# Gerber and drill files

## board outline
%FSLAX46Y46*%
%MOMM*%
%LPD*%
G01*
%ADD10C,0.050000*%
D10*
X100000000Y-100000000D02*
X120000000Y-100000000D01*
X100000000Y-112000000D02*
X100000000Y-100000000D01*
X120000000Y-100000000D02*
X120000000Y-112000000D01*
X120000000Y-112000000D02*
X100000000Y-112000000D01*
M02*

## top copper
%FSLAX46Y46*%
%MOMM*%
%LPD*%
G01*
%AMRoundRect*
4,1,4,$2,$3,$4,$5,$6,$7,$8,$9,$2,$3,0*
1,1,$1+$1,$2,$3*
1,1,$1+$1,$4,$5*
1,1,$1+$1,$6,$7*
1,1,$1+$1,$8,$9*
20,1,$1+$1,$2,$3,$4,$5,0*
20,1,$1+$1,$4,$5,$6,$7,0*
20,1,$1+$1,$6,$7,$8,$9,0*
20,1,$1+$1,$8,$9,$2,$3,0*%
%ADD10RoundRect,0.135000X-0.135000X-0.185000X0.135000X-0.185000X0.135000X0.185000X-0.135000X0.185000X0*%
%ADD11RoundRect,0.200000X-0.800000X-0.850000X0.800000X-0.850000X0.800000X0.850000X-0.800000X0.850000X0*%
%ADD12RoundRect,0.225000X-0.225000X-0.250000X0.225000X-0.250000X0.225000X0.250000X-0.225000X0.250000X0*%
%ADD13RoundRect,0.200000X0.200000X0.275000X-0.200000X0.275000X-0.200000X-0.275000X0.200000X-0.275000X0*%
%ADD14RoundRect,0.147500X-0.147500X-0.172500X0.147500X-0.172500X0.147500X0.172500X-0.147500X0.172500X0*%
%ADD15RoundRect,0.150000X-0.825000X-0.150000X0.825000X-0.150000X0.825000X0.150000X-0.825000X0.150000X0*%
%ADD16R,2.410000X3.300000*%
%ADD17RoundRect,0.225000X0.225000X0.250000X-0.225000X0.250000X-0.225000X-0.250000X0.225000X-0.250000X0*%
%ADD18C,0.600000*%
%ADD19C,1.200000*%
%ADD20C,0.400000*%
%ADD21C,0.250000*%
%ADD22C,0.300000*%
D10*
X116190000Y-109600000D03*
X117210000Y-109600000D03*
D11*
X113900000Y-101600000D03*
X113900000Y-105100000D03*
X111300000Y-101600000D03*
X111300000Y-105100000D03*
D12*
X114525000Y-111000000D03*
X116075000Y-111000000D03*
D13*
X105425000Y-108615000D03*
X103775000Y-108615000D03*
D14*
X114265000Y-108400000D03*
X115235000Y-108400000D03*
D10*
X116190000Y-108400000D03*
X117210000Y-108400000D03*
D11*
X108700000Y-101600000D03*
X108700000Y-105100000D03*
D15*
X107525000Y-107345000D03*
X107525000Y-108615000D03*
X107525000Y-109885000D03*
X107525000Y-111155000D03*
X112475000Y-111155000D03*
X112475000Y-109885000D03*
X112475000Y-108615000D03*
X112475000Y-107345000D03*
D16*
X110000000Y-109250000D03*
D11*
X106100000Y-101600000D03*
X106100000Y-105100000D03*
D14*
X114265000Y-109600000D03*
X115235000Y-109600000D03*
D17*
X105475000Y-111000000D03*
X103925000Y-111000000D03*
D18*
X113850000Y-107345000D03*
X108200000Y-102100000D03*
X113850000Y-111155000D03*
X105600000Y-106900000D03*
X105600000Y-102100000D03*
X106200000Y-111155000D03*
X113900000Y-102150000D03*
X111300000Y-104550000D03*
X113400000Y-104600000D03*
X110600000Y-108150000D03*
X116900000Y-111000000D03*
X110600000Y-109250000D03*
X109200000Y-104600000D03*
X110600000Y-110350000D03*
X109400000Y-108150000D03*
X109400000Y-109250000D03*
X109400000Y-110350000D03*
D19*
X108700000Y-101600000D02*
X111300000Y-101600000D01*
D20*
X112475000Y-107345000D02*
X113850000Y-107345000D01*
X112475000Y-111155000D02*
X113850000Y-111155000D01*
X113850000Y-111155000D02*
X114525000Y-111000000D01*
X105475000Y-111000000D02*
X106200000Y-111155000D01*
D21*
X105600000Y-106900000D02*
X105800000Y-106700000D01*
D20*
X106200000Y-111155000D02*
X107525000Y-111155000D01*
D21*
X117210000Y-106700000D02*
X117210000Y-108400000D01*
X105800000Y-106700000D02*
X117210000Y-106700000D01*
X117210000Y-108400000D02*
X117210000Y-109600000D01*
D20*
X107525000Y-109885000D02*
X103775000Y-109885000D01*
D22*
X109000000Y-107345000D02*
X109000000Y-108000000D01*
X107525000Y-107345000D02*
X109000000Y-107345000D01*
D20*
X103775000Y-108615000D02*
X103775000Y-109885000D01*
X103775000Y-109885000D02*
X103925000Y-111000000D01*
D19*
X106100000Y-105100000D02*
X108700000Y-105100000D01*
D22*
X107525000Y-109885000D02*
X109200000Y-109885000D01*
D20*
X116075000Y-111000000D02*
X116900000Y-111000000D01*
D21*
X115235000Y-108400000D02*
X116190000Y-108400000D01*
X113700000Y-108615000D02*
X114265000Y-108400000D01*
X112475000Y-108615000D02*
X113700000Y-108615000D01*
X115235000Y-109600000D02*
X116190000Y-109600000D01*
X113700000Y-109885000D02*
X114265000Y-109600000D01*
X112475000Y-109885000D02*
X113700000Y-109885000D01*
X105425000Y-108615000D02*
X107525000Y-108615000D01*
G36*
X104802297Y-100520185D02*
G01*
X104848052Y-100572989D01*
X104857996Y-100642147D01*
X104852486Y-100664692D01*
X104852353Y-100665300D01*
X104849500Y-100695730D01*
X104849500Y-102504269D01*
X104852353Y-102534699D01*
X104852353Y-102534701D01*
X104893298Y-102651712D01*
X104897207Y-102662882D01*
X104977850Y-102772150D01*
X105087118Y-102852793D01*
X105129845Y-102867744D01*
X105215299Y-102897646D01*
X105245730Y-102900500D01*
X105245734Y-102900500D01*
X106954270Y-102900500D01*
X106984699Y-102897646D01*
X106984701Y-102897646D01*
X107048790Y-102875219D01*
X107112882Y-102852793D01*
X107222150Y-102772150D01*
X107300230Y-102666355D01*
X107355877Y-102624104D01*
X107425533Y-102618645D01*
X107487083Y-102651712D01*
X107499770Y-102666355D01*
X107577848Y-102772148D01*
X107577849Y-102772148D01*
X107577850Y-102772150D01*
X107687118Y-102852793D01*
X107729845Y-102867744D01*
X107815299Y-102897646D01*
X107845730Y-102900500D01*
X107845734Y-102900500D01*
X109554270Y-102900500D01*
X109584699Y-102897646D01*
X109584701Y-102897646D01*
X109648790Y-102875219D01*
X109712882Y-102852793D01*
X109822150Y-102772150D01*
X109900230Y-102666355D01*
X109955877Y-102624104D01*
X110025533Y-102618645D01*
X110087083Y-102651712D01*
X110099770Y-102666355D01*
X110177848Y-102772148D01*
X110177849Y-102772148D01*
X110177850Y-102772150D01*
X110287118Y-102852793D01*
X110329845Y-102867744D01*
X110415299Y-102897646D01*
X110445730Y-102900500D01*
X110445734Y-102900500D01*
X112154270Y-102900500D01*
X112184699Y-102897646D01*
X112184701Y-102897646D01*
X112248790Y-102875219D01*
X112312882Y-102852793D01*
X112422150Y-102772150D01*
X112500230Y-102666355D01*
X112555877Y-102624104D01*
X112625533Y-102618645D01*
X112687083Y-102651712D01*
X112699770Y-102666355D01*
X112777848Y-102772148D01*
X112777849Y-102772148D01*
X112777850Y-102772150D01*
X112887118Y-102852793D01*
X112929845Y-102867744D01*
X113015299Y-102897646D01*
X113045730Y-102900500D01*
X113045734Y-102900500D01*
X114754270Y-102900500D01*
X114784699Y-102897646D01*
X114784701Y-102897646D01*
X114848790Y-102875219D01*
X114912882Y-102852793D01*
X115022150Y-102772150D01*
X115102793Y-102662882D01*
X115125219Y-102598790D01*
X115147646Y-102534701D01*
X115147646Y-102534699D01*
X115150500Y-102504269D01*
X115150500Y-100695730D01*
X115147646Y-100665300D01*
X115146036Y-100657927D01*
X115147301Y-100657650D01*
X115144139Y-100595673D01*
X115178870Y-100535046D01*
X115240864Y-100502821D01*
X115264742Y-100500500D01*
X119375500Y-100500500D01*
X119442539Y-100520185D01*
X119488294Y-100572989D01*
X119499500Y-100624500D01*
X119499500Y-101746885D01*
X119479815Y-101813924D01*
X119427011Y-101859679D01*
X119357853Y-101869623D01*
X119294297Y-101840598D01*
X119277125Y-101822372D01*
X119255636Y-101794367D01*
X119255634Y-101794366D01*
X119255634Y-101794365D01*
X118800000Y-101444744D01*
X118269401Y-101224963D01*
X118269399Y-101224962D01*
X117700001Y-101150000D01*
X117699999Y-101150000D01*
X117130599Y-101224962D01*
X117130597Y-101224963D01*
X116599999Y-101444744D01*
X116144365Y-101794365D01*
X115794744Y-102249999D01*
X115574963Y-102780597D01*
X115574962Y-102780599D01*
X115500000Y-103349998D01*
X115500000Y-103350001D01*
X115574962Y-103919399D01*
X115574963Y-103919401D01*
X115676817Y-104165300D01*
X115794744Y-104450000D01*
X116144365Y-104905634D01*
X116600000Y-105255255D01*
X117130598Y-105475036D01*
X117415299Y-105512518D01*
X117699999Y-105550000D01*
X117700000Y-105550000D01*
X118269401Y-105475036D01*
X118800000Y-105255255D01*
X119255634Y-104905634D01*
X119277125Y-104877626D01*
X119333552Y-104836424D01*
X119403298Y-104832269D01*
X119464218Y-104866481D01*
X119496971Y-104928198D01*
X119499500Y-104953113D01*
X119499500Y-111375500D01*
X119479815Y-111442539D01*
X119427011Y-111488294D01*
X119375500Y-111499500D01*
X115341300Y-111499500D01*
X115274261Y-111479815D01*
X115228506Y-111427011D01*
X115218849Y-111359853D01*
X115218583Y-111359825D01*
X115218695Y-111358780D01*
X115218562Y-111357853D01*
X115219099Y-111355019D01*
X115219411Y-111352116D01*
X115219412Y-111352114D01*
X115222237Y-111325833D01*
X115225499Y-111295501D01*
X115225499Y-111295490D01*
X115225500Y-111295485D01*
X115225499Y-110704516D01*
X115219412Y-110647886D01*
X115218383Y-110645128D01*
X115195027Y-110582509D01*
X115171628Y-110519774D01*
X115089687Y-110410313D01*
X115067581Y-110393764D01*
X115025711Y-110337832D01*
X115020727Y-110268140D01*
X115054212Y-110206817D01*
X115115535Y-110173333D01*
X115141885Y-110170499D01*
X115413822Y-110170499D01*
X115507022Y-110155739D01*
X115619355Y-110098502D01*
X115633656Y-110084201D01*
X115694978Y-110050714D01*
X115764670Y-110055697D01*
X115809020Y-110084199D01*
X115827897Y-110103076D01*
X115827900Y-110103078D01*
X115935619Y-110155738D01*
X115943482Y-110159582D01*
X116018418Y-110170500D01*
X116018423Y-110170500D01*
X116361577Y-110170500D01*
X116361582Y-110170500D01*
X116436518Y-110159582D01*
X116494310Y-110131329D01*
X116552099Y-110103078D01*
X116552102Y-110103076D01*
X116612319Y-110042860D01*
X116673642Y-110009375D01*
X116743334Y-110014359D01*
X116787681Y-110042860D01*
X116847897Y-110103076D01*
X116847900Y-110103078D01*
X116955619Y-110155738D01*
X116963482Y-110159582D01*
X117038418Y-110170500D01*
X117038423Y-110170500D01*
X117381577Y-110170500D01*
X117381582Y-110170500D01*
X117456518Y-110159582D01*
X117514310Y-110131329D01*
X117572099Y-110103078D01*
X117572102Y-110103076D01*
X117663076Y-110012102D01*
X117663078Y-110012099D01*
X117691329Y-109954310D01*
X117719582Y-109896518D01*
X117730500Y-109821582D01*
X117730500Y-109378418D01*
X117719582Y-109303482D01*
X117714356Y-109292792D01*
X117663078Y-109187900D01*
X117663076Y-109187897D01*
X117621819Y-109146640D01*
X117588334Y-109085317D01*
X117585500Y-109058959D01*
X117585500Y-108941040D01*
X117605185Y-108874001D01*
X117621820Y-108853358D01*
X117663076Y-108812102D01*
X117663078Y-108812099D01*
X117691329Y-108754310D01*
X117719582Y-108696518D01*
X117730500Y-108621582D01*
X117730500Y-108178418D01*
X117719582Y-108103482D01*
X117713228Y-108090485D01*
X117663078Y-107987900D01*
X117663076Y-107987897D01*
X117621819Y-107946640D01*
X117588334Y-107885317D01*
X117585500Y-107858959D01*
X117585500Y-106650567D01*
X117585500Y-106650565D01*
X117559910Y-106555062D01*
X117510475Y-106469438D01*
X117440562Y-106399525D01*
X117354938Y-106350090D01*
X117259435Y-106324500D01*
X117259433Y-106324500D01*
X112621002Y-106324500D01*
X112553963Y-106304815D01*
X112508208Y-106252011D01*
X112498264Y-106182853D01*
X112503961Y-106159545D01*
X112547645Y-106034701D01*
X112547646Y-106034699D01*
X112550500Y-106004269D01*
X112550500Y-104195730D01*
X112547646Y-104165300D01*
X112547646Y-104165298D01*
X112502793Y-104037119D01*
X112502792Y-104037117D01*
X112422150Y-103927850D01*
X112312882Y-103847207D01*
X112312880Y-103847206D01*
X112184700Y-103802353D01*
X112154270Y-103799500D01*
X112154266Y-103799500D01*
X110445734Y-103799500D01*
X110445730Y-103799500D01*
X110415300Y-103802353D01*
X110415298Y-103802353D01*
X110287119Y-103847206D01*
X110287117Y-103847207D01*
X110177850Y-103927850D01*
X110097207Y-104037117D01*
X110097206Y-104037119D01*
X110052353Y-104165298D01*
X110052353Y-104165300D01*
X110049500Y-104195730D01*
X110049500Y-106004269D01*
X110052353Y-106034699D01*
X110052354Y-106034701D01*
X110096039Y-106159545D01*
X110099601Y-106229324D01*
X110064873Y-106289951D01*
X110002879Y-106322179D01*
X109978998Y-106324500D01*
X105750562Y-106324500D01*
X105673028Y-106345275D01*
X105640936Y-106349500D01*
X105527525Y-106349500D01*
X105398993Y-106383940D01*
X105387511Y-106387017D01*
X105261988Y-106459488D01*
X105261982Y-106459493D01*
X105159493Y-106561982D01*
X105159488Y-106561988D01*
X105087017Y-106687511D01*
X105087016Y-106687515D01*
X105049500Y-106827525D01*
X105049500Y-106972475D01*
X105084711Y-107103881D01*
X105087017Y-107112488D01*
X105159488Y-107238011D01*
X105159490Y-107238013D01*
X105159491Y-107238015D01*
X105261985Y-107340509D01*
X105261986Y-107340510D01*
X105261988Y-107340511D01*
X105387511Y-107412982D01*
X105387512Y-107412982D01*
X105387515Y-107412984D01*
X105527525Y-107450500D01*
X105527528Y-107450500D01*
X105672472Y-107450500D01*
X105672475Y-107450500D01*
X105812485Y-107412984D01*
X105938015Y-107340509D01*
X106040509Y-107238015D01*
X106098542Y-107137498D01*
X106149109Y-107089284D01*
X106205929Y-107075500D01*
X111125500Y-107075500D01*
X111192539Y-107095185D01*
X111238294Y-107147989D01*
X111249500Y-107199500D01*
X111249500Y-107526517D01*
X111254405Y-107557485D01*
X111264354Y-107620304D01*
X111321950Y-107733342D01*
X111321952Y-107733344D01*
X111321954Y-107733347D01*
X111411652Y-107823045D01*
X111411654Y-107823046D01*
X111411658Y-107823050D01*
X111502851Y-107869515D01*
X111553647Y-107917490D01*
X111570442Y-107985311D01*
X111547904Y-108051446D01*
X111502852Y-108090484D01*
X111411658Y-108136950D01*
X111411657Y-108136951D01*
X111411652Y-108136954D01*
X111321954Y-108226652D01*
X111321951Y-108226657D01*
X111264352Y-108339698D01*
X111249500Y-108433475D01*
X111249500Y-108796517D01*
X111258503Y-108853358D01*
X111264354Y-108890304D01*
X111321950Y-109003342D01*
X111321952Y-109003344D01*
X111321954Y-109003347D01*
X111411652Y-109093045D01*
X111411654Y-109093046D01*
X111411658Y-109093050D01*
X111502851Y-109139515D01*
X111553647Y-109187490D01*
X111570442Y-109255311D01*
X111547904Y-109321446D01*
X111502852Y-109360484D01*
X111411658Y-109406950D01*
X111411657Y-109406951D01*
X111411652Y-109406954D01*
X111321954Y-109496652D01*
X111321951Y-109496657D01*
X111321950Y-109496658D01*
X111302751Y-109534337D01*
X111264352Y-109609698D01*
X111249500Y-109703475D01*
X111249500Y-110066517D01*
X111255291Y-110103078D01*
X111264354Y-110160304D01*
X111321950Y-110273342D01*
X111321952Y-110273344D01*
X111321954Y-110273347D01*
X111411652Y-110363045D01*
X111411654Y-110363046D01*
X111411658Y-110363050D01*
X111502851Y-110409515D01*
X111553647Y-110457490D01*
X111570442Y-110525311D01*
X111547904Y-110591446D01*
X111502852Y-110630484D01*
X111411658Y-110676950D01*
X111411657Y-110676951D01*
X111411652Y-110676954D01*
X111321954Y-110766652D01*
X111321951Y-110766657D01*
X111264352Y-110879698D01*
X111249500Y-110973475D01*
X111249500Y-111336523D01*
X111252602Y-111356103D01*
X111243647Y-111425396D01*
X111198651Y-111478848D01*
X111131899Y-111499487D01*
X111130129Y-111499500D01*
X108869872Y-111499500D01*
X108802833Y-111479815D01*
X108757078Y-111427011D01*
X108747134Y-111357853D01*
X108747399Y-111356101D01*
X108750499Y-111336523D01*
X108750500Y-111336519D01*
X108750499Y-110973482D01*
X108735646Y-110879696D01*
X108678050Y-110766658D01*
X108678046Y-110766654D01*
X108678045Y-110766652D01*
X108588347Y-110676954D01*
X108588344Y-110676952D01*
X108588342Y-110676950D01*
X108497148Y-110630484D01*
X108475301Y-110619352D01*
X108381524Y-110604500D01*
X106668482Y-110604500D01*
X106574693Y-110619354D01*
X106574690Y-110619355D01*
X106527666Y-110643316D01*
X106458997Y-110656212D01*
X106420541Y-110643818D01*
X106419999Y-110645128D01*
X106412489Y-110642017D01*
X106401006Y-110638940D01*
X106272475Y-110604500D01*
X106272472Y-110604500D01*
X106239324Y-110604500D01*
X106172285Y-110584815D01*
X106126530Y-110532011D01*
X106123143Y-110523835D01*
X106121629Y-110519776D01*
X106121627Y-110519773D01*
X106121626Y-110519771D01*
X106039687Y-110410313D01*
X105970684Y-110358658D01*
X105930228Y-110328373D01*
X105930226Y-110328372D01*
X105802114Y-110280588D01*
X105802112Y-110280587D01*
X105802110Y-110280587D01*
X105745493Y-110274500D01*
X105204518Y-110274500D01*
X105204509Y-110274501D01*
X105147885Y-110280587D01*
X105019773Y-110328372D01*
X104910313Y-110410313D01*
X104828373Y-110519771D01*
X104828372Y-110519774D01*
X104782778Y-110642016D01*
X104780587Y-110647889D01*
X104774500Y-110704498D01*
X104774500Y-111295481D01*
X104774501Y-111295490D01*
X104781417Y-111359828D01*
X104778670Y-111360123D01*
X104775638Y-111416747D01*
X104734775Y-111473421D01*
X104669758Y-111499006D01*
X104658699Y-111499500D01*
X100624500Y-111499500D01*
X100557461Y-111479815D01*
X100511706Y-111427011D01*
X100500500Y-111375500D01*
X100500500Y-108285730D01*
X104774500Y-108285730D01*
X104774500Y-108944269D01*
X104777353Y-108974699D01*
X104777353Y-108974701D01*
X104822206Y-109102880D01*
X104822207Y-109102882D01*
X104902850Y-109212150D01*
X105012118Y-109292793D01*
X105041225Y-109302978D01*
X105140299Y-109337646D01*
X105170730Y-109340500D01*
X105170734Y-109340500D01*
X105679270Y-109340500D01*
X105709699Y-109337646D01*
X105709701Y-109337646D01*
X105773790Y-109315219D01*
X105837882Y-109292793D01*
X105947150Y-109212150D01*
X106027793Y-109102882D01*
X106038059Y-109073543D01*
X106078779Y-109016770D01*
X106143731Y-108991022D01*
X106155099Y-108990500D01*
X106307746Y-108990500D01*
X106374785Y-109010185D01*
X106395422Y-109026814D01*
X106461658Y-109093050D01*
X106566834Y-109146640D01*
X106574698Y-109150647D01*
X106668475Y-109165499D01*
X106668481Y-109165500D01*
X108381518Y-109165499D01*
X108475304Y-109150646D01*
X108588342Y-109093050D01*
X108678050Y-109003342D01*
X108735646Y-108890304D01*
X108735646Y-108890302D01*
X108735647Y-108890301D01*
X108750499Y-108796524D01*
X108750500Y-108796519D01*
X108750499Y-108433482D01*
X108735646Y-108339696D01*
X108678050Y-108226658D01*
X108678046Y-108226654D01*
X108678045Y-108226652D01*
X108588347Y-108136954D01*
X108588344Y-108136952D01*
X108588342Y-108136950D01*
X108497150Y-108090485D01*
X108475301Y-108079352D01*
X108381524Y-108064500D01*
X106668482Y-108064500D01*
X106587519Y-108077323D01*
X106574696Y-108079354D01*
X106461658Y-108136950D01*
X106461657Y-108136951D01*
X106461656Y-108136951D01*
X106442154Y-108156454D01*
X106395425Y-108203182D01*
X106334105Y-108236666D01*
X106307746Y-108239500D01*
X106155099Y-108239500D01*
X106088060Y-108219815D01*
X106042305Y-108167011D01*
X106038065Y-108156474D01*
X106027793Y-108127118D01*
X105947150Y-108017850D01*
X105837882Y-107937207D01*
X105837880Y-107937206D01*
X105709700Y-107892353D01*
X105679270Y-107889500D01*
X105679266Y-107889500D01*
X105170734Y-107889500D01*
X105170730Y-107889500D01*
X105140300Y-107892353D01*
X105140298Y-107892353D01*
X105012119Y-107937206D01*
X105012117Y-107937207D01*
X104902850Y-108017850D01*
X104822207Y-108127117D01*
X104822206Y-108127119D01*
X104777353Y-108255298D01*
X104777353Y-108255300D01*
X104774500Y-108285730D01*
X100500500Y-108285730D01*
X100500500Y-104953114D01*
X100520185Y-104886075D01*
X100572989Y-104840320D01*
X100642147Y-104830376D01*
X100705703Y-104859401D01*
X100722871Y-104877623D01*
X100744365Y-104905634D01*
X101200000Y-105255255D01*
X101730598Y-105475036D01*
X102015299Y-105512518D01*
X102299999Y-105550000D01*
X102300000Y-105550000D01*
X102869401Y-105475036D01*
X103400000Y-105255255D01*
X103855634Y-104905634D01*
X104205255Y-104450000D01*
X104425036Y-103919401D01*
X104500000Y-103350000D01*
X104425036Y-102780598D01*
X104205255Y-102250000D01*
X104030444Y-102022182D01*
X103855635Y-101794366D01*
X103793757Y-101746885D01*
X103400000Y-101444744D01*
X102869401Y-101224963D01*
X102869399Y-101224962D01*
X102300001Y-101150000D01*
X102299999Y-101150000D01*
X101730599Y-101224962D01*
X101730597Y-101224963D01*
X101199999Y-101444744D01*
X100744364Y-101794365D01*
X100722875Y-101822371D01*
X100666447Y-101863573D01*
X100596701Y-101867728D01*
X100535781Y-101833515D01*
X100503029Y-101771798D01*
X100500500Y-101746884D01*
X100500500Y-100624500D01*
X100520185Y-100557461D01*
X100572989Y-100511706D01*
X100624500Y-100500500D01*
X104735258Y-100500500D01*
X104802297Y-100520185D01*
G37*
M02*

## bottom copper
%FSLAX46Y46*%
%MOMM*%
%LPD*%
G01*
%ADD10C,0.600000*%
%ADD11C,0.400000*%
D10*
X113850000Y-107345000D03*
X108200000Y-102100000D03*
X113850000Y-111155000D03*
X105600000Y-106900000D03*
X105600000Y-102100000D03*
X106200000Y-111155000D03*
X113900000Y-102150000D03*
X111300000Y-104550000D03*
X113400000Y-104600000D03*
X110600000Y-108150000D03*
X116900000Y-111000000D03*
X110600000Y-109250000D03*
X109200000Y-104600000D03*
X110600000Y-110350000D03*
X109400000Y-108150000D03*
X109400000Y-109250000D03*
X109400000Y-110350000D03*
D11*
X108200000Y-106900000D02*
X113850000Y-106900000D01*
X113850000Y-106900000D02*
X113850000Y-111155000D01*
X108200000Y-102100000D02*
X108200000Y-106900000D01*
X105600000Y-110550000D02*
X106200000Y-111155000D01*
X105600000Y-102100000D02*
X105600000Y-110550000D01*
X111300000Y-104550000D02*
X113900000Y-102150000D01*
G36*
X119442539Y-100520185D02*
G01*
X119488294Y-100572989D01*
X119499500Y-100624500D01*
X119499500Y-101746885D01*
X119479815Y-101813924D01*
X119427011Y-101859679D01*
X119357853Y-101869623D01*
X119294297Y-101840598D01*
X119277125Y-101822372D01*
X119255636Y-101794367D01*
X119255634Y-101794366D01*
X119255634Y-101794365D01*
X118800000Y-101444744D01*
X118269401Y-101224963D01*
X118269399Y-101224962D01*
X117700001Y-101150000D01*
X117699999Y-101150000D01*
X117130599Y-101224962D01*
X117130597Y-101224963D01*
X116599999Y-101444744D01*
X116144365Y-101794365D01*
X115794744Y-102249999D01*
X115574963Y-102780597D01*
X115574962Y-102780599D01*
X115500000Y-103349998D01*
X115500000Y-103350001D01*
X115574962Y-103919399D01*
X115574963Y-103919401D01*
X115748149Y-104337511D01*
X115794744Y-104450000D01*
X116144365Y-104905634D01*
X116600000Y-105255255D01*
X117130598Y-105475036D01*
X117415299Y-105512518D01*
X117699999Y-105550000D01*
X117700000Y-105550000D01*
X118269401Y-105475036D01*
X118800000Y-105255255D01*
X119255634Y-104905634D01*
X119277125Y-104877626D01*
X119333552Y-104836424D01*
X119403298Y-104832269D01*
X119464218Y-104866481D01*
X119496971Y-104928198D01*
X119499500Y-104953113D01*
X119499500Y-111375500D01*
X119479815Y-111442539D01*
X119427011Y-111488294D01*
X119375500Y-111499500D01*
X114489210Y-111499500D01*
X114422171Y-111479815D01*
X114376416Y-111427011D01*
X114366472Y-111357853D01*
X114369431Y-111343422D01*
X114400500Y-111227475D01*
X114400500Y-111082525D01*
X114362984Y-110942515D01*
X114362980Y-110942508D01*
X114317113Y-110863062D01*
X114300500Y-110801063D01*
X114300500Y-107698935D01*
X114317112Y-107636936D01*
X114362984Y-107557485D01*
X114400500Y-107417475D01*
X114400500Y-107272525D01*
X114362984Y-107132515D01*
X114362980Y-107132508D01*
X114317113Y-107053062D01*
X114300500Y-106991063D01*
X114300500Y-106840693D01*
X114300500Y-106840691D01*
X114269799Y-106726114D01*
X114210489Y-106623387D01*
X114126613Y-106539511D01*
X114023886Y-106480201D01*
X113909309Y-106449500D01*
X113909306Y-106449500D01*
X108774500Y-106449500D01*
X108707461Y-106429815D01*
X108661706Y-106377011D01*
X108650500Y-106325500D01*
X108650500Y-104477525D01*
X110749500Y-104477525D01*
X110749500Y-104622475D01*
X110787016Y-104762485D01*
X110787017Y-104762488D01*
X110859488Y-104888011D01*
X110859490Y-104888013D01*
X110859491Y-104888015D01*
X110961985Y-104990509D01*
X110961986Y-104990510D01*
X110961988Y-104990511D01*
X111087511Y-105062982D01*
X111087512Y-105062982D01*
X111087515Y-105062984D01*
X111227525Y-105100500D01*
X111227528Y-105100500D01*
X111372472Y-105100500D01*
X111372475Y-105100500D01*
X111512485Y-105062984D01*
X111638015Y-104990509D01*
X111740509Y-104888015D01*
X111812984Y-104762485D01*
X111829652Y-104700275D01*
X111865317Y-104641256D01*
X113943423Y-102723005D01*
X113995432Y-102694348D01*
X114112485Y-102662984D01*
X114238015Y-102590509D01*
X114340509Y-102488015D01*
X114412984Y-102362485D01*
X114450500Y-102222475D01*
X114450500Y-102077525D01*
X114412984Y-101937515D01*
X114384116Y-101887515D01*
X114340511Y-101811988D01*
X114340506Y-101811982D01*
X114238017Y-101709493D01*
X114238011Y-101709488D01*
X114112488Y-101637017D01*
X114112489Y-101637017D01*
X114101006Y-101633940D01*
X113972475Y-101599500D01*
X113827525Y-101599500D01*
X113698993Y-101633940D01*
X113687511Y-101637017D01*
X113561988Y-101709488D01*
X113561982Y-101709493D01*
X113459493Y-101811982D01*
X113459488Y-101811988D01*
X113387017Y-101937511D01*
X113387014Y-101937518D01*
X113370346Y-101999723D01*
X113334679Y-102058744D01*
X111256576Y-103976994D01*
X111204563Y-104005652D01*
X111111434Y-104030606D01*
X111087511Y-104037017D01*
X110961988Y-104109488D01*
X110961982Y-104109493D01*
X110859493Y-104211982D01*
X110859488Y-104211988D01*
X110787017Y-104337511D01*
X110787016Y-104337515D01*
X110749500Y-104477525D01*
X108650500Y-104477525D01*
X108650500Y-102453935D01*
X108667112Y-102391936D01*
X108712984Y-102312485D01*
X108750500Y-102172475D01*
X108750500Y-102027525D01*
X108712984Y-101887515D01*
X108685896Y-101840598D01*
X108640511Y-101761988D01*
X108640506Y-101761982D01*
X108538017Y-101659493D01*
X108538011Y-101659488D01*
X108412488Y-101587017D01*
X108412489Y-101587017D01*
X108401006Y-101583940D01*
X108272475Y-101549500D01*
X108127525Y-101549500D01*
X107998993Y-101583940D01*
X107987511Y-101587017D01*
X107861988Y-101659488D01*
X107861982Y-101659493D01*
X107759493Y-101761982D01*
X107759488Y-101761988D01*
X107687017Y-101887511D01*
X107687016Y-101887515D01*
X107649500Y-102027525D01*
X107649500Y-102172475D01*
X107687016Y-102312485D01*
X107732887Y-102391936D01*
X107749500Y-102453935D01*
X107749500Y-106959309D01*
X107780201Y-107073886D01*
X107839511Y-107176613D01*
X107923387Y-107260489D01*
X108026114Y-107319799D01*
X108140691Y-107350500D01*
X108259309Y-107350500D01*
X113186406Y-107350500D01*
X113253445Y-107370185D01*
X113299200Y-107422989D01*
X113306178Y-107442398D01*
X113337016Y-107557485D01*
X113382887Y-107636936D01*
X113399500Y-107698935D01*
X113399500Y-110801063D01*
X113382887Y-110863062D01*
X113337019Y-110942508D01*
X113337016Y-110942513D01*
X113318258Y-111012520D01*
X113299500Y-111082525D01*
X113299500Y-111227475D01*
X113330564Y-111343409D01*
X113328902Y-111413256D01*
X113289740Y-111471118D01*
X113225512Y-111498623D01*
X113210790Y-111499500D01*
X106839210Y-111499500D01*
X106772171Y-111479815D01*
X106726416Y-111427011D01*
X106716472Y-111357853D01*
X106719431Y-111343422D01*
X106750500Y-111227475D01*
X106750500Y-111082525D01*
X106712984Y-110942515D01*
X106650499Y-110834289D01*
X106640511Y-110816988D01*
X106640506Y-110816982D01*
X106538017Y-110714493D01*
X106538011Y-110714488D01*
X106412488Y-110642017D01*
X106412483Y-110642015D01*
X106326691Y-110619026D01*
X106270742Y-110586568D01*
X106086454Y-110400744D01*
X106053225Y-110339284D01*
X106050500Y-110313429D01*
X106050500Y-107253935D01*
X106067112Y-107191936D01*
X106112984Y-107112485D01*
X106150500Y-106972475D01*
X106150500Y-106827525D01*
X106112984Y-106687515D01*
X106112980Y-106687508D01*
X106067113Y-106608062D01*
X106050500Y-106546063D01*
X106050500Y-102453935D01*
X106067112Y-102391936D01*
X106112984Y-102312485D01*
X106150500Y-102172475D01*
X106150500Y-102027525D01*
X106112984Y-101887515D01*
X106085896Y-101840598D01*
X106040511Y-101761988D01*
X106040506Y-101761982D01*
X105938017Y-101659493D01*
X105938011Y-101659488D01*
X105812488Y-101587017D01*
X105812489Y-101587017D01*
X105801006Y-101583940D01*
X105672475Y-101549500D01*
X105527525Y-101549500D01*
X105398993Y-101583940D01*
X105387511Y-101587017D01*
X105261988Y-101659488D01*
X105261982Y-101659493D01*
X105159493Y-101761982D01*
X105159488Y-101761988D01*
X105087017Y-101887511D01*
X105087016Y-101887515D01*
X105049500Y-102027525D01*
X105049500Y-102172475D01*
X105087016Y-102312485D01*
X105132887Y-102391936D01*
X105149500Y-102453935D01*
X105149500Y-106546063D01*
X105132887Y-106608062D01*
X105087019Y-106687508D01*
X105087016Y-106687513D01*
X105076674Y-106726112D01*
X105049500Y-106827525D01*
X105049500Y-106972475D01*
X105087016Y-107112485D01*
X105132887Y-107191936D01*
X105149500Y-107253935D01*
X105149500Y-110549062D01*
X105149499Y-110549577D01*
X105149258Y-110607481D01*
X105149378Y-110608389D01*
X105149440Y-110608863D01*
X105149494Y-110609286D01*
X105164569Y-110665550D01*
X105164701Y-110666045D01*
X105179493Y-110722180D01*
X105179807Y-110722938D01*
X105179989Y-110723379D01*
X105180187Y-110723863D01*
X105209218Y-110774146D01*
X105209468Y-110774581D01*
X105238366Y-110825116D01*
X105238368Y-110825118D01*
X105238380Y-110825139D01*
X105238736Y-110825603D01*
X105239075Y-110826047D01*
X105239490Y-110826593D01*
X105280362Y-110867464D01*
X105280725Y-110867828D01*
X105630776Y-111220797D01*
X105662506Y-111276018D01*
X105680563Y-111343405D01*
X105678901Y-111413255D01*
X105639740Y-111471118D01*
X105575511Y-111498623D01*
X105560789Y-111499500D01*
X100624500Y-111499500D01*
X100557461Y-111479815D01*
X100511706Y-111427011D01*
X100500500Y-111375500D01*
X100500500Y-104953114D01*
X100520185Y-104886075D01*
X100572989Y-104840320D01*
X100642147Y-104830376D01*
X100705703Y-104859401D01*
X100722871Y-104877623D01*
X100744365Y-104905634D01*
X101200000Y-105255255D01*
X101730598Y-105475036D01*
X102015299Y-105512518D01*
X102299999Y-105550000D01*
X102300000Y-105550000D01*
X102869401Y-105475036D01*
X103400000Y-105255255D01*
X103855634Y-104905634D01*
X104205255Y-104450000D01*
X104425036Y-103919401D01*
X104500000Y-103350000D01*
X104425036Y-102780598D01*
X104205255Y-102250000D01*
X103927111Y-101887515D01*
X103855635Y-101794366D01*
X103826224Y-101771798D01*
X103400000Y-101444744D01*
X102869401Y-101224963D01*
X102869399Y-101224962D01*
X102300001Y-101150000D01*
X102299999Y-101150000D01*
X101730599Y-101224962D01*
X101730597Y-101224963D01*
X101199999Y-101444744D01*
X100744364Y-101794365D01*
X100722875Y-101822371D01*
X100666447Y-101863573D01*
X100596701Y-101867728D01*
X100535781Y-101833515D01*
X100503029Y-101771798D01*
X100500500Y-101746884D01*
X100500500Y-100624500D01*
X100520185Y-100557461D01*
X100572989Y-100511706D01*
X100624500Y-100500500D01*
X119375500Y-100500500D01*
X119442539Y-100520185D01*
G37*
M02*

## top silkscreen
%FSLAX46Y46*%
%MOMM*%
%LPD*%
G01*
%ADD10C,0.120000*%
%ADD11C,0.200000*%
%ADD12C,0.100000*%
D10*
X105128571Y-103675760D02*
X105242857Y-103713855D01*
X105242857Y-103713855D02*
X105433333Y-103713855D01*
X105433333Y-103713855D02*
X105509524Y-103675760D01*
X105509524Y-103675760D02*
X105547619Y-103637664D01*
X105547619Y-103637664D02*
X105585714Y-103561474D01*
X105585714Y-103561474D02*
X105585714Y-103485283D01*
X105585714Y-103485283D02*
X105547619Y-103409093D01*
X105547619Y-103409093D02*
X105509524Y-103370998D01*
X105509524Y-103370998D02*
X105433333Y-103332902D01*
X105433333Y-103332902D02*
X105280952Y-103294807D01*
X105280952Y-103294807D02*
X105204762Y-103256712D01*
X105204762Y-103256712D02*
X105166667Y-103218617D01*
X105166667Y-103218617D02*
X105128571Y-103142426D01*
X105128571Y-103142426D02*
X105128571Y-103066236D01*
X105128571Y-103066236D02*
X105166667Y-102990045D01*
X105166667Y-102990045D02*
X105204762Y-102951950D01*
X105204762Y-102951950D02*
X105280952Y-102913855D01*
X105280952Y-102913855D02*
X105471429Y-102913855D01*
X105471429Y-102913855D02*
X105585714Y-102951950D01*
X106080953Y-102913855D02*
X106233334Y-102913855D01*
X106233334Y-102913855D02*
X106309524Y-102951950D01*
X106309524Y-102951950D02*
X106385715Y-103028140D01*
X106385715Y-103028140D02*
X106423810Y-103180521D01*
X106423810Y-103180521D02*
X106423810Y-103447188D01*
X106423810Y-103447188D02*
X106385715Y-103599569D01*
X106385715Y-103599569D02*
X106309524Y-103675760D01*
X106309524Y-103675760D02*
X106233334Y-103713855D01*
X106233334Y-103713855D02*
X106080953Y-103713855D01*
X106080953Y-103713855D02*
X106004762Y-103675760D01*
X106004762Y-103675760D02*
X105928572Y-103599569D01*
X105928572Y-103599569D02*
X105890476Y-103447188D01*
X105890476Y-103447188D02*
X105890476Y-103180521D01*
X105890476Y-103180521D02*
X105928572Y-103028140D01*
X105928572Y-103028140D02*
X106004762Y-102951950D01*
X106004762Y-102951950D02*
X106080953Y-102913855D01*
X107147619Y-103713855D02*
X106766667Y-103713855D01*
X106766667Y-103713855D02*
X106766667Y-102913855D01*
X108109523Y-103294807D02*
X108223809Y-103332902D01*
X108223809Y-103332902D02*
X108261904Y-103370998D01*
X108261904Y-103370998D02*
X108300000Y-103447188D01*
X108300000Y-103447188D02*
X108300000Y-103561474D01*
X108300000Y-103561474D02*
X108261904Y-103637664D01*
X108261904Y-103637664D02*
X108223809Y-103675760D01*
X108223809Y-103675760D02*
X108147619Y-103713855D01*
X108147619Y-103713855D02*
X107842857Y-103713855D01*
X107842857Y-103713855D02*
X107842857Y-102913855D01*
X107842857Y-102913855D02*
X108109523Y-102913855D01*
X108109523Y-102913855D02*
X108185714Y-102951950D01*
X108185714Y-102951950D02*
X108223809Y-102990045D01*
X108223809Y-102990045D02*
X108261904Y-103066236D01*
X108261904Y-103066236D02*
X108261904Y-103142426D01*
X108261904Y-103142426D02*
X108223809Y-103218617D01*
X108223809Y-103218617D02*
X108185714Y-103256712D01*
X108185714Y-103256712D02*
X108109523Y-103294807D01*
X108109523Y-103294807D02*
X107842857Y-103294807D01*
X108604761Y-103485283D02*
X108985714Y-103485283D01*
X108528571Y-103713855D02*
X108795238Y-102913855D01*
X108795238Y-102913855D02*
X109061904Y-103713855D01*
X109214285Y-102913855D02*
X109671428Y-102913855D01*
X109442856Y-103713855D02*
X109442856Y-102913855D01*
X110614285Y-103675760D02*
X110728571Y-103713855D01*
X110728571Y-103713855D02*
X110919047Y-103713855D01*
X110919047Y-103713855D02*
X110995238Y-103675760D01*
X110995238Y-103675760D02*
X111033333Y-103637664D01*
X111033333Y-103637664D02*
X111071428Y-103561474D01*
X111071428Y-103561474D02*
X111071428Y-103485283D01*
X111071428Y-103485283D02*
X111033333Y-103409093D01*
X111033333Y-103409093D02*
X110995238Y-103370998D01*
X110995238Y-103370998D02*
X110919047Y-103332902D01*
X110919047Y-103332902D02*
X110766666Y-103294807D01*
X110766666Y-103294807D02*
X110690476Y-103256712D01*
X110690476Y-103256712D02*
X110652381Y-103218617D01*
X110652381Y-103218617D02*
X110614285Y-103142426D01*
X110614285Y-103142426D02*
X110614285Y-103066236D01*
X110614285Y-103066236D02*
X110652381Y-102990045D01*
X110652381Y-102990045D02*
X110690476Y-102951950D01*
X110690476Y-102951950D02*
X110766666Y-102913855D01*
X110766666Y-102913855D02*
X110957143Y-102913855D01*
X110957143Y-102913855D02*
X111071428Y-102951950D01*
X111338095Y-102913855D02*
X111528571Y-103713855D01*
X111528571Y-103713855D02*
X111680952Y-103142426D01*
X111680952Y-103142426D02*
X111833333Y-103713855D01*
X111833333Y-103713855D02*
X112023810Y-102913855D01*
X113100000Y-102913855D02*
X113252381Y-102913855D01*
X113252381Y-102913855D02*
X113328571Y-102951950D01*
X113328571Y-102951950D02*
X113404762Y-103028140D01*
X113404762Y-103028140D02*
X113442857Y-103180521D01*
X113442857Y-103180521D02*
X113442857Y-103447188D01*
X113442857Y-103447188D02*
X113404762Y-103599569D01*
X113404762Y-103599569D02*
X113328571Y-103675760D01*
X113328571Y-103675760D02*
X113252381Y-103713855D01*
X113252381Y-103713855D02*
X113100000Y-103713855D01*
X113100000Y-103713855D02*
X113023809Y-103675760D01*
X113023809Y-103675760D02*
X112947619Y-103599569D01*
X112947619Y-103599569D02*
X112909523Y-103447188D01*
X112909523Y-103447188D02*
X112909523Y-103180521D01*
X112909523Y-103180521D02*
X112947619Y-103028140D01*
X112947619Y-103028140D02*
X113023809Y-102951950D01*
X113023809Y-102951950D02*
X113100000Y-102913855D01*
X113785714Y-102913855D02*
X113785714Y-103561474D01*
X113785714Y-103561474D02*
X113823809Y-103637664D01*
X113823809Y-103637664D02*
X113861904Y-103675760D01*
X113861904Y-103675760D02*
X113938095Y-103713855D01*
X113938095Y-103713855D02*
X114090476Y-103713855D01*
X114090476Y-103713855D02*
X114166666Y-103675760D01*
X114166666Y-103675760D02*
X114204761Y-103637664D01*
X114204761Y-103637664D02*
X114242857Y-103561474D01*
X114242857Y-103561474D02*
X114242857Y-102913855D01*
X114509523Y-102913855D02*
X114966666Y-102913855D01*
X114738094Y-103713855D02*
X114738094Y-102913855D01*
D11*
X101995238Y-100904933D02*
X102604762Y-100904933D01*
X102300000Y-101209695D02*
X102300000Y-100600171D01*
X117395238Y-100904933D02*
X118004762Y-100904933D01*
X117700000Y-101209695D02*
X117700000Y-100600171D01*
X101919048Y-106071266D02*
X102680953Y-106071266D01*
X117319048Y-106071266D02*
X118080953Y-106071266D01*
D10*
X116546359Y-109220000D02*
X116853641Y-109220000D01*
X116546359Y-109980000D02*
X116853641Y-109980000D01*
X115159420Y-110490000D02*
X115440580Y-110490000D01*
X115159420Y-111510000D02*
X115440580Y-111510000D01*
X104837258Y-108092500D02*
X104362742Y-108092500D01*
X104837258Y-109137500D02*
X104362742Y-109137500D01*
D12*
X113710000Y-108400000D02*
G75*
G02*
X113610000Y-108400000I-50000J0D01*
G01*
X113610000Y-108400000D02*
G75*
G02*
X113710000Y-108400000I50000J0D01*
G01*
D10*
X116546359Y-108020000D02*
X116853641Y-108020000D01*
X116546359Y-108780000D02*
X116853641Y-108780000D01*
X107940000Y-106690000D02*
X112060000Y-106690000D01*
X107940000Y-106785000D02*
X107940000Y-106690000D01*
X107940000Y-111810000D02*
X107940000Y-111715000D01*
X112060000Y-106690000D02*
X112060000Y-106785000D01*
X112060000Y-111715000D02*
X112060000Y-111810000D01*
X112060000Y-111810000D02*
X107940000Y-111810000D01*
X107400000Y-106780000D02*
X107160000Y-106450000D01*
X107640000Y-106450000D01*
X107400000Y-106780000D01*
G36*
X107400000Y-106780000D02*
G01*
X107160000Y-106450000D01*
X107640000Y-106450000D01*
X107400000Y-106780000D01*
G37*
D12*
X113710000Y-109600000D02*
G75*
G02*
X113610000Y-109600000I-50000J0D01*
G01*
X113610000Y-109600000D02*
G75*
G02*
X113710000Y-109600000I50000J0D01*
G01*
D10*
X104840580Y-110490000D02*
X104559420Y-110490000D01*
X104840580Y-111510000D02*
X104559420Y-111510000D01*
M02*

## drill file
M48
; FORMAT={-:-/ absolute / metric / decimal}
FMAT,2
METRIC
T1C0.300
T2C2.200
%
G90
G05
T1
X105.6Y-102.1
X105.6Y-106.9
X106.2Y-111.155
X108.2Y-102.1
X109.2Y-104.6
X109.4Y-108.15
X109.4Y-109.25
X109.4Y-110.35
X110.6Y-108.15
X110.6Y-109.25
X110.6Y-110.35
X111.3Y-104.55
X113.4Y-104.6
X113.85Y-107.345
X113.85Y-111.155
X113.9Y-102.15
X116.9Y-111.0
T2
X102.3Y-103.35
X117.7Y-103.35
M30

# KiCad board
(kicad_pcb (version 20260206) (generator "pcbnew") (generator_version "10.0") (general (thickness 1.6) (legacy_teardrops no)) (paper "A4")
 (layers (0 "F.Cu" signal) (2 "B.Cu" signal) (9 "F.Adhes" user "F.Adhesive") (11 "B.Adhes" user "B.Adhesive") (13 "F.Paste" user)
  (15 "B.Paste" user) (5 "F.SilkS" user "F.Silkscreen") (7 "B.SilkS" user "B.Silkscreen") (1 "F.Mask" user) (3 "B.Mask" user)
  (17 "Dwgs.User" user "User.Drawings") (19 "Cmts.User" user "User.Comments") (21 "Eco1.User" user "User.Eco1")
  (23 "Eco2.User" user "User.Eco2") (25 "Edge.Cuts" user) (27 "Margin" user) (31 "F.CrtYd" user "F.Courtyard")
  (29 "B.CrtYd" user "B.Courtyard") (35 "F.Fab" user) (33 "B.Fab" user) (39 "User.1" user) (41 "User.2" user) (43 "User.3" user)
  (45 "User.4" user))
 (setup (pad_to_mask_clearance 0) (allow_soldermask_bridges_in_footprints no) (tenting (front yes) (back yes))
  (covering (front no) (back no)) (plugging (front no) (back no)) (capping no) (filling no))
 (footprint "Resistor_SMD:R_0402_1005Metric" (layer "F.Cu") (at 116.7 109.6)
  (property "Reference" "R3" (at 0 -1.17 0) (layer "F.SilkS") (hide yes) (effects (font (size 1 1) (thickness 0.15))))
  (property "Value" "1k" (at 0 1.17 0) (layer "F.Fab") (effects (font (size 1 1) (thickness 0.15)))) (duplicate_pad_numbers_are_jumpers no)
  (fp_line (start -0.153641 -0.38) (end 0.153641 -0.38) (stroke (width 0.12) (type solid)) (layer "F.SilkS"))
  (fp_line (start -0.153641 0.38) (end 0.153641 0.38) (stroke (width 0.12) (type solid)) (layer "F.SilkS"))
  (pad "1" smd roundrect (at -0.51 0) (size 0.54 0.64) (layers "F.Cu" "F.Mask" "F.Paste") (roundrect_rratio 0.25) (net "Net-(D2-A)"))
  (pad "2" smd roundrect (at 0.51 0) (size 0.54 0.64) (layers "F.Cu" "F.Mask" "F.Paste") (roundrect_rratio 0.25) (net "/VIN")))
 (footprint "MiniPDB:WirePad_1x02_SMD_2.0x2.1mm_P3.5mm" (layer "F.Cu") (at 113.9 103.35)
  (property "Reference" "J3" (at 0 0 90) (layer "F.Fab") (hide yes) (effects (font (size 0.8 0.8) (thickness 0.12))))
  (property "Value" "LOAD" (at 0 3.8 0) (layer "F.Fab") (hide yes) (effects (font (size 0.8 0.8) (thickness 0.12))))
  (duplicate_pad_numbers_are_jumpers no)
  (pad "1" smd roundrect (at 0 -1.75) (size 2 2.1) (layers "F.Cu" "F.Mask") (roundrect_rratio 0.1) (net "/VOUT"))
  (pad "2" smd roundrect (at 0 1.75) (size 2 2.1) (layers "F.Cu" "F.Mask") (roundrect_rratio 0.1) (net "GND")))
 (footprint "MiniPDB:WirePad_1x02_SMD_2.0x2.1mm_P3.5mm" (layer "F.Cu") (at 111.3 103.35)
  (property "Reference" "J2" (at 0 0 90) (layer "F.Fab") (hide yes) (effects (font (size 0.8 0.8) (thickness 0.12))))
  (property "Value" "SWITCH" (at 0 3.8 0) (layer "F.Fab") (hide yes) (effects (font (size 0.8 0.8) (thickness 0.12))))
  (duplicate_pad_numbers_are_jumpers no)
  (pad "1" smd roundrect (at 0 -1.75) (size 2 2.1) (layers "F.Cu" "F.Mask") (roundrect_rratio 0.1) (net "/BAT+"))
  (pad "2" smd roundrect (at 0 1.75) (size 2 2.1) (layers "F.Cu" "F.Mask") (roundrect_rratio 0.1) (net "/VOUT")))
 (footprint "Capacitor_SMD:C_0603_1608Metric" (layer "F.Cu") (at 115.3 111)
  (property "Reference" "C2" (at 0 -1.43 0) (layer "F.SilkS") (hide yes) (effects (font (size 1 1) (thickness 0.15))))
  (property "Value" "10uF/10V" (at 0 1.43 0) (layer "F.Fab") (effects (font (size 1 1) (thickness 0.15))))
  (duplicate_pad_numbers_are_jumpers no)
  (fp_line (start -0.14058 -0.51) (end 0.14058 -0.51) (stroke (width 0.12) (type solid)) (layer "F.SilkS"))
  (fp_line (start -0.14058 0.51) (end 0.14058 0.51) (stroke (width 0.12) (type solid)) (layer "F.SilkS"))
  (pad "1" smd roundrect (at -0.775 0) (size 0.9 0.95) (layers "F.Cu" "F.Mask" "F.Paste") (roundrect_rratio 0.25) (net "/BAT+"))
  (pad "2" smd roundrect (at 0.775 0) (size 0.9 0.95) (layers "F.Cu" "F.Mask" "F.Paste") (roundrect_rratio 0.25) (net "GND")))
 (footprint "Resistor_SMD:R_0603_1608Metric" (layer "F.Cu") (at 104.6 108.615 180)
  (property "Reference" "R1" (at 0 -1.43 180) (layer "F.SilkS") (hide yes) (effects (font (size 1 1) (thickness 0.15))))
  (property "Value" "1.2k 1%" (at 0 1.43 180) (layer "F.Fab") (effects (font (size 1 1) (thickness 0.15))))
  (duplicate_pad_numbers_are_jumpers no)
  (fp_line (start -0.237258 0.5225) (end 0.237258 0.5225) (stroke (width 0.12) (type solid)) (layer "F.SilkS"))
  (fp_line (start -0.237258 -0.5225) (end 0.237258 -0.5225) (stroke (width 0.12) (type solid)) (layer "F.SilkS"))
  (pad "1" smd roundrect (at -0.825 0 180) (size 0.8 0.95) (layers "F.Cu" "F.Mask" "F.Paste") (roundrect_rratio 0.25) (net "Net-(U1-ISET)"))
  (pad "2" smd roundrect (at 0.825 0 180) (size 0.8 0.95) (layers "F.Cu" "F.Mask" "F.Paste") (roundrect_rratio 0.25) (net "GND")))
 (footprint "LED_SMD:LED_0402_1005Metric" (layer "F.Cu") (at 114.75 108.4)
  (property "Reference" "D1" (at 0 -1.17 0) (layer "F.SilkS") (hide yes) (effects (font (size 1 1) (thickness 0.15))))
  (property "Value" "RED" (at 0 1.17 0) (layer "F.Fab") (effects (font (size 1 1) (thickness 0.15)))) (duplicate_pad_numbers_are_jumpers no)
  (fp_circle (center -1.09 0) (end -1.04 0) (stroke (width 0.1) (type solid)) (fill no) (layer "F.SilkS"))
  (pad "1" smd roundrect (at -0.485 0) (size 0.59 0.64) (layers "F.Cu" "F.Mask" "F.Paste") (roundrect_rratio 0.25) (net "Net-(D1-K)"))
  (pad "2" smd roundrect (at 0.485 0) (size 0.59 0.64) (layers "F.Cu" "F.Mask" "F.Paste") (roundrect_rratio 0.25) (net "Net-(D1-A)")))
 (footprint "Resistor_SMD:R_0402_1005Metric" (layer "F.Cu") (at 116.7 108.4)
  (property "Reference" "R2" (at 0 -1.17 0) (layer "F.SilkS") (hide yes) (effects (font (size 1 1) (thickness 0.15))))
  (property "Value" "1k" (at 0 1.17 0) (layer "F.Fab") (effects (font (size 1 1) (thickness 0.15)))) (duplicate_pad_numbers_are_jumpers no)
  (fp_line (start -0.153641 -0.38) (end 0.153641 -0.38) (stroke (width 0.12) (type solid)) (layer "F.SilkS"))
  (fp_line (start -0.153641 0.38) (end 0.153641 0.38) (stroke (width 0.12) (type solid)) (layer "F.SilkS"))
  (pad "1" smd roundrect (at -0.51 0) (size 0.54 0.64) (layers "F.Cu" "F.Mask" "F.Paste") (roundrect_rratio 0.25) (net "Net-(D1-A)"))
  (pad "2" smd roundrect (at 0.51 0) (size 0.54 0.64) (layers "F.Cu" "F.Mask" "F.Paste") (roundrect_rratio 0.25) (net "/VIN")))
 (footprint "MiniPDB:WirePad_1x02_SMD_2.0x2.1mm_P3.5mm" (layer "F.Cu") (at 108.7 103.35)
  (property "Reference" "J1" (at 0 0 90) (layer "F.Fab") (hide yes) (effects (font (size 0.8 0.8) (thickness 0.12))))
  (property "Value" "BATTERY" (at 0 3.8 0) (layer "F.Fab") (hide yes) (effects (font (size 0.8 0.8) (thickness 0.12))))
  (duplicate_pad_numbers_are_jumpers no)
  (pad "1" smd roundrect (at 0 -1.75) (size 2 2.1) (layers "F.Cu" "F.Mask") (roundrect_rratio 0.1) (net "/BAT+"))
  (pad "2" smd roundrect (at 0 1.75) (size 2 2.1) (layers "F.Cu" "F.Mask") (roundrect_rratio 0.1) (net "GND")))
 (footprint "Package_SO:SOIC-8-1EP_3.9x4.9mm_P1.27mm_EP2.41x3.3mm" (layer "F.Cu") (at 110 109.25)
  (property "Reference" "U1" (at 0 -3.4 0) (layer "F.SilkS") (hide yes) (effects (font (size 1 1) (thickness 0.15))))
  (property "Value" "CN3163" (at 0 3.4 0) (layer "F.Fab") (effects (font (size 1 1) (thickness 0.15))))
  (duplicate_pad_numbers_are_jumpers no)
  (fp_line (start -2.06 -2.56) (end 2.06 -2.56) (stroke (width 0.12) (type solid)) (layer "F.SilkS"))
  (fp_line (start -2.06 -2.465) (end -2.06 -2.56) (stroke (width 0.12) (type solid)) (layer "F.SilkS"))
  (fp_line (start -2.06 2.56) (end -2.06 2.465) (stroke (width 0.12) (type solid)) (layer "F.SilkS"))
  (fp_line (start 2.06 -2.56) (end 2.06 -2.465) (stroke (width 0.12) (type solid)) (layer "F.SilkS"))
  (fp_line (start 2.06 2.465) (end 2.06 2.56) (stroke (width 0.12) (type solid)) (layer "F.SilkS"))
  (fp_line (start 2.06 2.56) (end -2.06 2.56) (stroke (width 0.12) (type solid)) (layer "F.SilkS"))
  (fp_poly (pts (xy -2.6 -2.47) (xy -2.84 -2.8) (xy -2.36 -2.8)) (stroke (width 0.12) (type solid)) (fill yes) (layer "F.SilkS"))
  (pad "" smd roundrect (at -0.6 -0.825) (size 0.97 1.33) (layers "F.Paste") (roundrect_rratio 0.25))
  (pad "" smd roundrect (at -0.6 0.825) (size 0.97 1.33) (layers "F.Paste") (roundrect_rratio 0.25))
  (pad "" smd roundrect (at 0.6 -0.825) (size 0.97 1.33) (layers "F.Paste") (roundrect_rratio 0.25))
  (pad "" smd roundrect (at 0.6 0.825) (size 0.97 1.33) (layers "F.Paste") (roundrect_rratio 0.25))
  (pad "1" smd roundrect (at -2.475 -1.905) (size 1.95 0.6) (layers "F.Cu" "F.Mask" "F.Paste") (roundrect_rratio 0.25) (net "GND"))
  (pad "2" smd roundrect (at -2.475 -0.635) (size 1.95 0.6) (layers "F.Cu" "F.Mask" "F.Paste") (roundrect_rratio 0.25) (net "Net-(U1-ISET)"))
  (pad "3" smd roundrect (at -2.475 0.635) (size 1.95 0.6) (layers "F.Cu" "F.Mask" "F.Paste") (roundrect_rratio 0.25) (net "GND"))
  (pad "4" smd roundrect (at -2.475 1.905) (size 1.95 0.6) (layers "F.Cu" "F.Mask" "F.Paste") (roundrect_rratio 0.25) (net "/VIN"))
  (pad "5" smd roundrect (at 2.475 1.905) (size 1.95 0.6) (layers "F.Cu" "F.Mask" "F.Paste") (roundrect_rratio 0.25) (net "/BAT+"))
  (pad "6" smd roundrect (at 2.475 0.635) (size 1.95 0.6) (layers "F.Cu" "F.Mask" "F.Paste") (roundrect_rratio 0.25) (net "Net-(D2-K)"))
  (pad "7" smd roundrect (at 2.475 -0.635) (size 1.95 0.6) (layers "F.Cu" "F.Mask" "F.Paste") (roundrect_rratio 0.25) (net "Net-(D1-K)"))
  (pad "8" smd roundrect (at 2.475 -1.905) (size 1.95 0.6) (layers "F.Cu" "F.Mask" "F.Paste") (roundrect_rratio 0.25) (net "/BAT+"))
  (pad "9" smd rect (at 0 0) (size 2.41 3.3) (layers "F.Cu" "F.Mask") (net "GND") (zone_connect 2)))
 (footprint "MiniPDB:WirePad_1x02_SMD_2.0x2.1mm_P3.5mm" (layer "F.Cu") (at 106.1 103.35)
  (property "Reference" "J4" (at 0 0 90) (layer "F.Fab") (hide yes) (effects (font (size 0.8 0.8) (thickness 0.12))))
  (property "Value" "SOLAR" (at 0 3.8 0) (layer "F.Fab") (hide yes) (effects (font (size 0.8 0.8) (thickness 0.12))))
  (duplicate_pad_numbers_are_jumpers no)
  (pad "1" smd roundrect (at 0 -1.75) (size 2 2.1) (layers "F.Cu" "F.Mask") (roundrect_rratio 0.1) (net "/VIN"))
  (pad "2" smd roundrect (at 0 1.75) (size 2 2.1) (layers "F.Cu" "F.Mask") (roundrect_rratio 0.1) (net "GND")))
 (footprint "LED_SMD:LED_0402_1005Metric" (layer "F.Cu") (at 114.75 109.6)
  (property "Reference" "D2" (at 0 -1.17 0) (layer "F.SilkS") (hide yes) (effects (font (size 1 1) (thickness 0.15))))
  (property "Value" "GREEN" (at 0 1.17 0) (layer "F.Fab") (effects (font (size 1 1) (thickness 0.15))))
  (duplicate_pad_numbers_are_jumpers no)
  (fp_circle (center -1.09 0) (end -1.04 0) (stroke (width 0.1) (type solid)) (fill no) (layer "F.SilkS"))
  (pad "1" smd roundrect (at -0.485 0) (size 0.59 0.64) (layers "F.Cu" "F.Mask" "F.Paste") (roundrect_rratio 0.25) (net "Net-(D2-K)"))
  (pad "2" smd roundrect (at 0.485 0) (size 0.59 0.64) (layers "F.Cu" "F.Mask" "F.Paste") (roundrect_rratio 0.25) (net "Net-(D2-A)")))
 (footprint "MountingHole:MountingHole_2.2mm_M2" (layer "F.Cu") (at 102.3 103.35)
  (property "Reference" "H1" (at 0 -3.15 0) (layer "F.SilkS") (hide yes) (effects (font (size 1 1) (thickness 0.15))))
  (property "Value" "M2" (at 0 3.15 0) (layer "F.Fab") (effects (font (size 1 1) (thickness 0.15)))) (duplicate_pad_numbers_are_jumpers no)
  (pad "" np_thru_hole circle (at 0 0) (size 2.2 2.2) (drill 2.2) (layers "*.Cu" "*.Mask")))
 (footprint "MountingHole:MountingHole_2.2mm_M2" (layer "F.Cu") (at 117.7 103.35)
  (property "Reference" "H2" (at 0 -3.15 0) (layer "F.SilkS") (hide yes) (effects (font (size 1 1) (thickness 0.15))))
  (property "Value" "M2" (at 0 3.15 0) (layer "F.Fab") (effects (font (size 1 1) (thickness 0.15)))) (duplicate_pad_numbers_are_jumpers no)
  (pad "" np_thru_hole circle (at 0 0) (size 2.2 2.2) (drill 2.2) (layers "*.Cu" "*.Mask")))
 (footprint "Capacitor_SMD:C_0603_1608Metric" (layer "F.Cu") (at 104.7 111 180)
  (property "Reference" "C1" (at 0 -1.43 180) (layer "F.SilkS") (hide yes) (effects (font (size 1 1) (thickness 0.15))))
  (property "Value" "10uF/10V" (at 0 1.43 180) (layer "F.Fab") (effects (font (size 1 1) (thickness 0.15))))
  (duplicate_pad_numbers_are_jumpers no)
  (fp_line (start -0.14058 0.51) (end 0.14058 0.51) (stroke (width 0.12) (type solid)) (layer "F.SilkS"))
  (fp_line (start -0.14058 -0.51) (end 0.14058 -0.51) (stroke (width 0.12) (type solid)) (layer "F.SilkS"))
  (pad "1" smd roundrect (at -0.775 0 180) (size 0.9 0.95) (layers "F.Cu" "F.Mask" "F.Paste") (roundrect_rratio 0.25) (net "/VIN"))
  (pad "2" smd roundrect (at 0.775 0 180) (size 0.9 0.95) (layers "F.Cu" "F.Mask" "F.Paste") (roundrect_rratio 0.25) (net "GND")))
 (gr_line (start 100 100) (end 120 100) (stroke (width 0.05) (type default)) (layer "Edge.Cuts"))
 (gr_line (start 100 112) (end 100 100) (stroke (width 0.05) (type default)) (layer "Edge.Cuts"))
 (gr_line (start 120 100) (end 120 112) (stroke (width 0.05) (type default)) (layer "Edge.Cuts"))
 (gr_line (start 120 112) (end 100 112) (stroke (width 0.05) (type default)) (layer "Edge.Cuts"))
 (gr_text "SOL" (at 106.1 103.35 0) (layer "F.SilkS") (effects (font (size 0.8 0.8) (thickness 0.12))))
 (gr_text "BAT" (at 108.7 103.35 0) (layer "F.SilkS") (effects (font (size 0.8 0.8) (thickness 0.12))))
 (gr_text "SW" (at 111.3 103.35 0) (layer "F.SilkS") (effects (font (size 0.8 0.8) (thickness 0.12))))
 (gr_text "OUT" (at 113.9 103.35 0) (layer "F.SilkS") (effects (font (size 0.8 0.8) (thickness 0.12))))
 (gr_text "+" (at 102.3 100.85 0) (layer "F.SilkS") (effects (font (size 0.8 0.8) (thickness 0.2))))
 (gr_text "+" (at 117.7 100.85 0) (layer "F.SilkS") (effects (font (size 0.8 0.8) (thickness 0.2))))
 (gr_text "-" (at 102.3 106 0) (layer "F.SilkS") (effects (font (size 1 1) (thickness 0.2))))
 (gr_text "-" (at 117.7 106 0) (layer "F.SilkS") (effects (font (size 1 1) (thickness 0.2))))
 (segment (start 108.7 101.6) (end 111.3 101.6) (width 1.2) (layer "F.Cu") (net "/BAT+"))
 (segment (start 112.475 107.345) (end 113.85 107.345) (width 0.4) (layer "F.Cu") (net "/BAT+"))
 (segment (start 112.475 111.155) (end 113.85 111.155) (width 0.4) (layer "F.Cu") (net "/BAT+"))
 (segment (start 113.85 111.155) (end 114.525 111) (width 0.4) (layer "F.Cu") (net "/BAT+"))
 (via (at 113.85 107.345) (size 0.6) (drill 0.3) (layers "F.Cu" "B.Cu") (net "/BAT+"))
 (via (at 108.2 102.1) (size 0.6) (drill 0.3) (layers "F.Cu" "B.Cu") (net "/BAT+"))
 (via (at 113.85 111.155) (size 0.6) (drill 0.3) (layers "F.Cu" "B.Cu") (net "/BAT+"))
 (segment (start 108.2 106.9) (end 113.85 106.9) (width 0.4) (layer "B.Cu") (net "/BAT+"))
 (segment (start 113.85 106.9) (end 113.85 111.155) (width 0.4) (layer "B.Cu") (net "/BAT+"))
 (segment (start 108.2 102.1) (end 108.2 106.9) (width 0.4) (layer "B.Cu") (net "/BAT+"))
 (segment (start 105.475 111) (end 106.2 111.155) (width 0.4) (layer "F.Cu") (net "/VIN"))
 (segment (start 105.6 106.9) (end 105.8 106.7) (width 0.25) (layer "F.Cu") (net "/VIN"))
 (segment (start 106.2 111.155) (end 107.525 111.155) (width 0.4) (layer "F.Cu") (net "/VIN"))
 (segment (start 117.21 106.7) (end 117.21 108.4) (width 0.25) (layer "F.Cu") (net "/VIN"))
 (segment (start 105.8 106.7) (end 117.21 106.7) (width 0.25) (layer "F.Cu") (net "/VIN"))
 (segment (start 117.21 108.4) (end 117.21 109.6) (width 0.25) (layer "F.Cu") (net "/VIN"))
 (via (at 105.6 106.9) (size 0.6) (drill 0.3) (layers "F.Cu" "B.Cu") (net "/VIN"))
 (via (at 105.6 102.1) (size 0.6) (drill 0.3) (layers "F.Cu" "B.Cu") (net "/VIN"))
 (via (at 106.2 111.155) (size 0.6) (drill 0.3) (layers "F.Cu" "B.Cu") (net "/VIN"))
 (segment (start 105.6 110.55) (end 106.2 111.155) (width 0.4) (layer "B.Cu") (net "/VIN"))
 (segment (start 105.6 102.1) (end 105.6 110.55) (width 0.4) (layer "B.Cu") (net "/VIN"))
 (via (at 113.9 102.15) (size 0.6) (drill 0.3) (layers "F.Cu" "B.Cu") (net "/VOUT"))
 (via (at 111.3 104.55) (size 0.6) (drill 0.3) (layers "F.Cu" "B.Cu") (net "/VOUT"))
 (segment (start 111.3 104.55) (end 113.9 102.15) (width 0.4) (layer "B.Cu") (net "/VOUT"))
 (segment (start 107.525 109.885) (end 103.775 109.885) (width 0.4) (layer "F.Cu") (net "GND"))
 (segment (start 109 107.345) (end 109 108) (width 0.3) (layer "F.Cu") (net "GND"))
 (segment (start 107.525 107.345) (end 109 107.345) (width 0.3) (layer "F.Cu") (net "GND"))
 (segment (start 103.775 108.615) (end 103.775 109.885) (width 0.4) (layer "F.Cu") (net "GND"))
 (segment (start 103.775 109.885) (end 103.925 111) (width 0.4) (layer "F.Cu") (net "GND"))
 (segment (start 106.1 105.1) (end 108.7 105.1) (width 1.2) (layer "F.Cu") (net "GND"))
 (segment (start 107.525 109.885) (end 109.2 109.885) (width 0.3) (layer "F.Cu") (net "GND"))
 (segment (start 116.075 111) (end 116.9 111) (width 0.4) (layer "F.Cu") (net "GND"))
 (via (at 113.4 104.6) (size 0.6) (drill 0.3) (layers "F.Cu" "B.Cu") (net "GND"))
 (via (at 110.6 108.15) (size 0.6) (drill 0.3) (layers "F.Cu" "B.Cu") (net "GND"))
 (via (at 116.9 111) (size 0.6) (drill 0.3) (layers "F.Cu" "B.Cu") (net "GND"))
 (via (at 110.6 109.25) (size 0.6) (drill 0.3) (layers "F.Cu" "B.Cu") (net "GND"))
 (via (at 109.2 104.6) (size 0.6) (drill 0.3) (layers "F.Cu" "B.Cu") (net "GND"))
 (via (at 110.6 110.35) (size 0.6) (drill 0.3) (layers "F.Cu" "B.Cu") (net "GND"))
 (via (at 109.4 108.15) (size 0.6) (drill 0.3) (layers "F.Cu" "B.Cu") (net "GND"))
 (via (at 109.4 109.25) (size 0.6) (drill 0.3) (layers "F.Cu" "B.Cu") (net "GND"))
 (via (at 109.4 110.35) (size 0.6) (drill 0.3) (layers "F.Cu" "B.Cu") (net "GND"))
 (segment (start 115.235 108.4) (end 116.19 108.4) (width 0.25) (layer "F.Cu") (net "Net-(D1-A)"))
 (segment (start 113.7 108.615) (end 114.265 108.4) (width 0.25) (layer "F.Cu") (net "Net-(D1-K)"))
 (segment (start 112.475 108.615) (end 113.7 108.615) (width 0.25) (layer "F.Cu") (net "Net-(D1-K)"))
 (segment (start 115.235 109.6) (end 116.19 109.6) (width 0.25) (layer "F.Cu") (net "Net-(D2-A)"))
 (segment (start 113.7 109.885) (end 114.265 109.6) (width 0.25) (layer "F.Cu") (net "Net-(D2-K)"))
 (segment (start 112.475 109.885) (end 113.7 109.885) (width 0.25) (layer "F.Cu") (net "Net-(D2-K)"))
 (segment (start 105.425 108.615) (end 107.525 108.615) (width 0.25) (layer "F.Cu") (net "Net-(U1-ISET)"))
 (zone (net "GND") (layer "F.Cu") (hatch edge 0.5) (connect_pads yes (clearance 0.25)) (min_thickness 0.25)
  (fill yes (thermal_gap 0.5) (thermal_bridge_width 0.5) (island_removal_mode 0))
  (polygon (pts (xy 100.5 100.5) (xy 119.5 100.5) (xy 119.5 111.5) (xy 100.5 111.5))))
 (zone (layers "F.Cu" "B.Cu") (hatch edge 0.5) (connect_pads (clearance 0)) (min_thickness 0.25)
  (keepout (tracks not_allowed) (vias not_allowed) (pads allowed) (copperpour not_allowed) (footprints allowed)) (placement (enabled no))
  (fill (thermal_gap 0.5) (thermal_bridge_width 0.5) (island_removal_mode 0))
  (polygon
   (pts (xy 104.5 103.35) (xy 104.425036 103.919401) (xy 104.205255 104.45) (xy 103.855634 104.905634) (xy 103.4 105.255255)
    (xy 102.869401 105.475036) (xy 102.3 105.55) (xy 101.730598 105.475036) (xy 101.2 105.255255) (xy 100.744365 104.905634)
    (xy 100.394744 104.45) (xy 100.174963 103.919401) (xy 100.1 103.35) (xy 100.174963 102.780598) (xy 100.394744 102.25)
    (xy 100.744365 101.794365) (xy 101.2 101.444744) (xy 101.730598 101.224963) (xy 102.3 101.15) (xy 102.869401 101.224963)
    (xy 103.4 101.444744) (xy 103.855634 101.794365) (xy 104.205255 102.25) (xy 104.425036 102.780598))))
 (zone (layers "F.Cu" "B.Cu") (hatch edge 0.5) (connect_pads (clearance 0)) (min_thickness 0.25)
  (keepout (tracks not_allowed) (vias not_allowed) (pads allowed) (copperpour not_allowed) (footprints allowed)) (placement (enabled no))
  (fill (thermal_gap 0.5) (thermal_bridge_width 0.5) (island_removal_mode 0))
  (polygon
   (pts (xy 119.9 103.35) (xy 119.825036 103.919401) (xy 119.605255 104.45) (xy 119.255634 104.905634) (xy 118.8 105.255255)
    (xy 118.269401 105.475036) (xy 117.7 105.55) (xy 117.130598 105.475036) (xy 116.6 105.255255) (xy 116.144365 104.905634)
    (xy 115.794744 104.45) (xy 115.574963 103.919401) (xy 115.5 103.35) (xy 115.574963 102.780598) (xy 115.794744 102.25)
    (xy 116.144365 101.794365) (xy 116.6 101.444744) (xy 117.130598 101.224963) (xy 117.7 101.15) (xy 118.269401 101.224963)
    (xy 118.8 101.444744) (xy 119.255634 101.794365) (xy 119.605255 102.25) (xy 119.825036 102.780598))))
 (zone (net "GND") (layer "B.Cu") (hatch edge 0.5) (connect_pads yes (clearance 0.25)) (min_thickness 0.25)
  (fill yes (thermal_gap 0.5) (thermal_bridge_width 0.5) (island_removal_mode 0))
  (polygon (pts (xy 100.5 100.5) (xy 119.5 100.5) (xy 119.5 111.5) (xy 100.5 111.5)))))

